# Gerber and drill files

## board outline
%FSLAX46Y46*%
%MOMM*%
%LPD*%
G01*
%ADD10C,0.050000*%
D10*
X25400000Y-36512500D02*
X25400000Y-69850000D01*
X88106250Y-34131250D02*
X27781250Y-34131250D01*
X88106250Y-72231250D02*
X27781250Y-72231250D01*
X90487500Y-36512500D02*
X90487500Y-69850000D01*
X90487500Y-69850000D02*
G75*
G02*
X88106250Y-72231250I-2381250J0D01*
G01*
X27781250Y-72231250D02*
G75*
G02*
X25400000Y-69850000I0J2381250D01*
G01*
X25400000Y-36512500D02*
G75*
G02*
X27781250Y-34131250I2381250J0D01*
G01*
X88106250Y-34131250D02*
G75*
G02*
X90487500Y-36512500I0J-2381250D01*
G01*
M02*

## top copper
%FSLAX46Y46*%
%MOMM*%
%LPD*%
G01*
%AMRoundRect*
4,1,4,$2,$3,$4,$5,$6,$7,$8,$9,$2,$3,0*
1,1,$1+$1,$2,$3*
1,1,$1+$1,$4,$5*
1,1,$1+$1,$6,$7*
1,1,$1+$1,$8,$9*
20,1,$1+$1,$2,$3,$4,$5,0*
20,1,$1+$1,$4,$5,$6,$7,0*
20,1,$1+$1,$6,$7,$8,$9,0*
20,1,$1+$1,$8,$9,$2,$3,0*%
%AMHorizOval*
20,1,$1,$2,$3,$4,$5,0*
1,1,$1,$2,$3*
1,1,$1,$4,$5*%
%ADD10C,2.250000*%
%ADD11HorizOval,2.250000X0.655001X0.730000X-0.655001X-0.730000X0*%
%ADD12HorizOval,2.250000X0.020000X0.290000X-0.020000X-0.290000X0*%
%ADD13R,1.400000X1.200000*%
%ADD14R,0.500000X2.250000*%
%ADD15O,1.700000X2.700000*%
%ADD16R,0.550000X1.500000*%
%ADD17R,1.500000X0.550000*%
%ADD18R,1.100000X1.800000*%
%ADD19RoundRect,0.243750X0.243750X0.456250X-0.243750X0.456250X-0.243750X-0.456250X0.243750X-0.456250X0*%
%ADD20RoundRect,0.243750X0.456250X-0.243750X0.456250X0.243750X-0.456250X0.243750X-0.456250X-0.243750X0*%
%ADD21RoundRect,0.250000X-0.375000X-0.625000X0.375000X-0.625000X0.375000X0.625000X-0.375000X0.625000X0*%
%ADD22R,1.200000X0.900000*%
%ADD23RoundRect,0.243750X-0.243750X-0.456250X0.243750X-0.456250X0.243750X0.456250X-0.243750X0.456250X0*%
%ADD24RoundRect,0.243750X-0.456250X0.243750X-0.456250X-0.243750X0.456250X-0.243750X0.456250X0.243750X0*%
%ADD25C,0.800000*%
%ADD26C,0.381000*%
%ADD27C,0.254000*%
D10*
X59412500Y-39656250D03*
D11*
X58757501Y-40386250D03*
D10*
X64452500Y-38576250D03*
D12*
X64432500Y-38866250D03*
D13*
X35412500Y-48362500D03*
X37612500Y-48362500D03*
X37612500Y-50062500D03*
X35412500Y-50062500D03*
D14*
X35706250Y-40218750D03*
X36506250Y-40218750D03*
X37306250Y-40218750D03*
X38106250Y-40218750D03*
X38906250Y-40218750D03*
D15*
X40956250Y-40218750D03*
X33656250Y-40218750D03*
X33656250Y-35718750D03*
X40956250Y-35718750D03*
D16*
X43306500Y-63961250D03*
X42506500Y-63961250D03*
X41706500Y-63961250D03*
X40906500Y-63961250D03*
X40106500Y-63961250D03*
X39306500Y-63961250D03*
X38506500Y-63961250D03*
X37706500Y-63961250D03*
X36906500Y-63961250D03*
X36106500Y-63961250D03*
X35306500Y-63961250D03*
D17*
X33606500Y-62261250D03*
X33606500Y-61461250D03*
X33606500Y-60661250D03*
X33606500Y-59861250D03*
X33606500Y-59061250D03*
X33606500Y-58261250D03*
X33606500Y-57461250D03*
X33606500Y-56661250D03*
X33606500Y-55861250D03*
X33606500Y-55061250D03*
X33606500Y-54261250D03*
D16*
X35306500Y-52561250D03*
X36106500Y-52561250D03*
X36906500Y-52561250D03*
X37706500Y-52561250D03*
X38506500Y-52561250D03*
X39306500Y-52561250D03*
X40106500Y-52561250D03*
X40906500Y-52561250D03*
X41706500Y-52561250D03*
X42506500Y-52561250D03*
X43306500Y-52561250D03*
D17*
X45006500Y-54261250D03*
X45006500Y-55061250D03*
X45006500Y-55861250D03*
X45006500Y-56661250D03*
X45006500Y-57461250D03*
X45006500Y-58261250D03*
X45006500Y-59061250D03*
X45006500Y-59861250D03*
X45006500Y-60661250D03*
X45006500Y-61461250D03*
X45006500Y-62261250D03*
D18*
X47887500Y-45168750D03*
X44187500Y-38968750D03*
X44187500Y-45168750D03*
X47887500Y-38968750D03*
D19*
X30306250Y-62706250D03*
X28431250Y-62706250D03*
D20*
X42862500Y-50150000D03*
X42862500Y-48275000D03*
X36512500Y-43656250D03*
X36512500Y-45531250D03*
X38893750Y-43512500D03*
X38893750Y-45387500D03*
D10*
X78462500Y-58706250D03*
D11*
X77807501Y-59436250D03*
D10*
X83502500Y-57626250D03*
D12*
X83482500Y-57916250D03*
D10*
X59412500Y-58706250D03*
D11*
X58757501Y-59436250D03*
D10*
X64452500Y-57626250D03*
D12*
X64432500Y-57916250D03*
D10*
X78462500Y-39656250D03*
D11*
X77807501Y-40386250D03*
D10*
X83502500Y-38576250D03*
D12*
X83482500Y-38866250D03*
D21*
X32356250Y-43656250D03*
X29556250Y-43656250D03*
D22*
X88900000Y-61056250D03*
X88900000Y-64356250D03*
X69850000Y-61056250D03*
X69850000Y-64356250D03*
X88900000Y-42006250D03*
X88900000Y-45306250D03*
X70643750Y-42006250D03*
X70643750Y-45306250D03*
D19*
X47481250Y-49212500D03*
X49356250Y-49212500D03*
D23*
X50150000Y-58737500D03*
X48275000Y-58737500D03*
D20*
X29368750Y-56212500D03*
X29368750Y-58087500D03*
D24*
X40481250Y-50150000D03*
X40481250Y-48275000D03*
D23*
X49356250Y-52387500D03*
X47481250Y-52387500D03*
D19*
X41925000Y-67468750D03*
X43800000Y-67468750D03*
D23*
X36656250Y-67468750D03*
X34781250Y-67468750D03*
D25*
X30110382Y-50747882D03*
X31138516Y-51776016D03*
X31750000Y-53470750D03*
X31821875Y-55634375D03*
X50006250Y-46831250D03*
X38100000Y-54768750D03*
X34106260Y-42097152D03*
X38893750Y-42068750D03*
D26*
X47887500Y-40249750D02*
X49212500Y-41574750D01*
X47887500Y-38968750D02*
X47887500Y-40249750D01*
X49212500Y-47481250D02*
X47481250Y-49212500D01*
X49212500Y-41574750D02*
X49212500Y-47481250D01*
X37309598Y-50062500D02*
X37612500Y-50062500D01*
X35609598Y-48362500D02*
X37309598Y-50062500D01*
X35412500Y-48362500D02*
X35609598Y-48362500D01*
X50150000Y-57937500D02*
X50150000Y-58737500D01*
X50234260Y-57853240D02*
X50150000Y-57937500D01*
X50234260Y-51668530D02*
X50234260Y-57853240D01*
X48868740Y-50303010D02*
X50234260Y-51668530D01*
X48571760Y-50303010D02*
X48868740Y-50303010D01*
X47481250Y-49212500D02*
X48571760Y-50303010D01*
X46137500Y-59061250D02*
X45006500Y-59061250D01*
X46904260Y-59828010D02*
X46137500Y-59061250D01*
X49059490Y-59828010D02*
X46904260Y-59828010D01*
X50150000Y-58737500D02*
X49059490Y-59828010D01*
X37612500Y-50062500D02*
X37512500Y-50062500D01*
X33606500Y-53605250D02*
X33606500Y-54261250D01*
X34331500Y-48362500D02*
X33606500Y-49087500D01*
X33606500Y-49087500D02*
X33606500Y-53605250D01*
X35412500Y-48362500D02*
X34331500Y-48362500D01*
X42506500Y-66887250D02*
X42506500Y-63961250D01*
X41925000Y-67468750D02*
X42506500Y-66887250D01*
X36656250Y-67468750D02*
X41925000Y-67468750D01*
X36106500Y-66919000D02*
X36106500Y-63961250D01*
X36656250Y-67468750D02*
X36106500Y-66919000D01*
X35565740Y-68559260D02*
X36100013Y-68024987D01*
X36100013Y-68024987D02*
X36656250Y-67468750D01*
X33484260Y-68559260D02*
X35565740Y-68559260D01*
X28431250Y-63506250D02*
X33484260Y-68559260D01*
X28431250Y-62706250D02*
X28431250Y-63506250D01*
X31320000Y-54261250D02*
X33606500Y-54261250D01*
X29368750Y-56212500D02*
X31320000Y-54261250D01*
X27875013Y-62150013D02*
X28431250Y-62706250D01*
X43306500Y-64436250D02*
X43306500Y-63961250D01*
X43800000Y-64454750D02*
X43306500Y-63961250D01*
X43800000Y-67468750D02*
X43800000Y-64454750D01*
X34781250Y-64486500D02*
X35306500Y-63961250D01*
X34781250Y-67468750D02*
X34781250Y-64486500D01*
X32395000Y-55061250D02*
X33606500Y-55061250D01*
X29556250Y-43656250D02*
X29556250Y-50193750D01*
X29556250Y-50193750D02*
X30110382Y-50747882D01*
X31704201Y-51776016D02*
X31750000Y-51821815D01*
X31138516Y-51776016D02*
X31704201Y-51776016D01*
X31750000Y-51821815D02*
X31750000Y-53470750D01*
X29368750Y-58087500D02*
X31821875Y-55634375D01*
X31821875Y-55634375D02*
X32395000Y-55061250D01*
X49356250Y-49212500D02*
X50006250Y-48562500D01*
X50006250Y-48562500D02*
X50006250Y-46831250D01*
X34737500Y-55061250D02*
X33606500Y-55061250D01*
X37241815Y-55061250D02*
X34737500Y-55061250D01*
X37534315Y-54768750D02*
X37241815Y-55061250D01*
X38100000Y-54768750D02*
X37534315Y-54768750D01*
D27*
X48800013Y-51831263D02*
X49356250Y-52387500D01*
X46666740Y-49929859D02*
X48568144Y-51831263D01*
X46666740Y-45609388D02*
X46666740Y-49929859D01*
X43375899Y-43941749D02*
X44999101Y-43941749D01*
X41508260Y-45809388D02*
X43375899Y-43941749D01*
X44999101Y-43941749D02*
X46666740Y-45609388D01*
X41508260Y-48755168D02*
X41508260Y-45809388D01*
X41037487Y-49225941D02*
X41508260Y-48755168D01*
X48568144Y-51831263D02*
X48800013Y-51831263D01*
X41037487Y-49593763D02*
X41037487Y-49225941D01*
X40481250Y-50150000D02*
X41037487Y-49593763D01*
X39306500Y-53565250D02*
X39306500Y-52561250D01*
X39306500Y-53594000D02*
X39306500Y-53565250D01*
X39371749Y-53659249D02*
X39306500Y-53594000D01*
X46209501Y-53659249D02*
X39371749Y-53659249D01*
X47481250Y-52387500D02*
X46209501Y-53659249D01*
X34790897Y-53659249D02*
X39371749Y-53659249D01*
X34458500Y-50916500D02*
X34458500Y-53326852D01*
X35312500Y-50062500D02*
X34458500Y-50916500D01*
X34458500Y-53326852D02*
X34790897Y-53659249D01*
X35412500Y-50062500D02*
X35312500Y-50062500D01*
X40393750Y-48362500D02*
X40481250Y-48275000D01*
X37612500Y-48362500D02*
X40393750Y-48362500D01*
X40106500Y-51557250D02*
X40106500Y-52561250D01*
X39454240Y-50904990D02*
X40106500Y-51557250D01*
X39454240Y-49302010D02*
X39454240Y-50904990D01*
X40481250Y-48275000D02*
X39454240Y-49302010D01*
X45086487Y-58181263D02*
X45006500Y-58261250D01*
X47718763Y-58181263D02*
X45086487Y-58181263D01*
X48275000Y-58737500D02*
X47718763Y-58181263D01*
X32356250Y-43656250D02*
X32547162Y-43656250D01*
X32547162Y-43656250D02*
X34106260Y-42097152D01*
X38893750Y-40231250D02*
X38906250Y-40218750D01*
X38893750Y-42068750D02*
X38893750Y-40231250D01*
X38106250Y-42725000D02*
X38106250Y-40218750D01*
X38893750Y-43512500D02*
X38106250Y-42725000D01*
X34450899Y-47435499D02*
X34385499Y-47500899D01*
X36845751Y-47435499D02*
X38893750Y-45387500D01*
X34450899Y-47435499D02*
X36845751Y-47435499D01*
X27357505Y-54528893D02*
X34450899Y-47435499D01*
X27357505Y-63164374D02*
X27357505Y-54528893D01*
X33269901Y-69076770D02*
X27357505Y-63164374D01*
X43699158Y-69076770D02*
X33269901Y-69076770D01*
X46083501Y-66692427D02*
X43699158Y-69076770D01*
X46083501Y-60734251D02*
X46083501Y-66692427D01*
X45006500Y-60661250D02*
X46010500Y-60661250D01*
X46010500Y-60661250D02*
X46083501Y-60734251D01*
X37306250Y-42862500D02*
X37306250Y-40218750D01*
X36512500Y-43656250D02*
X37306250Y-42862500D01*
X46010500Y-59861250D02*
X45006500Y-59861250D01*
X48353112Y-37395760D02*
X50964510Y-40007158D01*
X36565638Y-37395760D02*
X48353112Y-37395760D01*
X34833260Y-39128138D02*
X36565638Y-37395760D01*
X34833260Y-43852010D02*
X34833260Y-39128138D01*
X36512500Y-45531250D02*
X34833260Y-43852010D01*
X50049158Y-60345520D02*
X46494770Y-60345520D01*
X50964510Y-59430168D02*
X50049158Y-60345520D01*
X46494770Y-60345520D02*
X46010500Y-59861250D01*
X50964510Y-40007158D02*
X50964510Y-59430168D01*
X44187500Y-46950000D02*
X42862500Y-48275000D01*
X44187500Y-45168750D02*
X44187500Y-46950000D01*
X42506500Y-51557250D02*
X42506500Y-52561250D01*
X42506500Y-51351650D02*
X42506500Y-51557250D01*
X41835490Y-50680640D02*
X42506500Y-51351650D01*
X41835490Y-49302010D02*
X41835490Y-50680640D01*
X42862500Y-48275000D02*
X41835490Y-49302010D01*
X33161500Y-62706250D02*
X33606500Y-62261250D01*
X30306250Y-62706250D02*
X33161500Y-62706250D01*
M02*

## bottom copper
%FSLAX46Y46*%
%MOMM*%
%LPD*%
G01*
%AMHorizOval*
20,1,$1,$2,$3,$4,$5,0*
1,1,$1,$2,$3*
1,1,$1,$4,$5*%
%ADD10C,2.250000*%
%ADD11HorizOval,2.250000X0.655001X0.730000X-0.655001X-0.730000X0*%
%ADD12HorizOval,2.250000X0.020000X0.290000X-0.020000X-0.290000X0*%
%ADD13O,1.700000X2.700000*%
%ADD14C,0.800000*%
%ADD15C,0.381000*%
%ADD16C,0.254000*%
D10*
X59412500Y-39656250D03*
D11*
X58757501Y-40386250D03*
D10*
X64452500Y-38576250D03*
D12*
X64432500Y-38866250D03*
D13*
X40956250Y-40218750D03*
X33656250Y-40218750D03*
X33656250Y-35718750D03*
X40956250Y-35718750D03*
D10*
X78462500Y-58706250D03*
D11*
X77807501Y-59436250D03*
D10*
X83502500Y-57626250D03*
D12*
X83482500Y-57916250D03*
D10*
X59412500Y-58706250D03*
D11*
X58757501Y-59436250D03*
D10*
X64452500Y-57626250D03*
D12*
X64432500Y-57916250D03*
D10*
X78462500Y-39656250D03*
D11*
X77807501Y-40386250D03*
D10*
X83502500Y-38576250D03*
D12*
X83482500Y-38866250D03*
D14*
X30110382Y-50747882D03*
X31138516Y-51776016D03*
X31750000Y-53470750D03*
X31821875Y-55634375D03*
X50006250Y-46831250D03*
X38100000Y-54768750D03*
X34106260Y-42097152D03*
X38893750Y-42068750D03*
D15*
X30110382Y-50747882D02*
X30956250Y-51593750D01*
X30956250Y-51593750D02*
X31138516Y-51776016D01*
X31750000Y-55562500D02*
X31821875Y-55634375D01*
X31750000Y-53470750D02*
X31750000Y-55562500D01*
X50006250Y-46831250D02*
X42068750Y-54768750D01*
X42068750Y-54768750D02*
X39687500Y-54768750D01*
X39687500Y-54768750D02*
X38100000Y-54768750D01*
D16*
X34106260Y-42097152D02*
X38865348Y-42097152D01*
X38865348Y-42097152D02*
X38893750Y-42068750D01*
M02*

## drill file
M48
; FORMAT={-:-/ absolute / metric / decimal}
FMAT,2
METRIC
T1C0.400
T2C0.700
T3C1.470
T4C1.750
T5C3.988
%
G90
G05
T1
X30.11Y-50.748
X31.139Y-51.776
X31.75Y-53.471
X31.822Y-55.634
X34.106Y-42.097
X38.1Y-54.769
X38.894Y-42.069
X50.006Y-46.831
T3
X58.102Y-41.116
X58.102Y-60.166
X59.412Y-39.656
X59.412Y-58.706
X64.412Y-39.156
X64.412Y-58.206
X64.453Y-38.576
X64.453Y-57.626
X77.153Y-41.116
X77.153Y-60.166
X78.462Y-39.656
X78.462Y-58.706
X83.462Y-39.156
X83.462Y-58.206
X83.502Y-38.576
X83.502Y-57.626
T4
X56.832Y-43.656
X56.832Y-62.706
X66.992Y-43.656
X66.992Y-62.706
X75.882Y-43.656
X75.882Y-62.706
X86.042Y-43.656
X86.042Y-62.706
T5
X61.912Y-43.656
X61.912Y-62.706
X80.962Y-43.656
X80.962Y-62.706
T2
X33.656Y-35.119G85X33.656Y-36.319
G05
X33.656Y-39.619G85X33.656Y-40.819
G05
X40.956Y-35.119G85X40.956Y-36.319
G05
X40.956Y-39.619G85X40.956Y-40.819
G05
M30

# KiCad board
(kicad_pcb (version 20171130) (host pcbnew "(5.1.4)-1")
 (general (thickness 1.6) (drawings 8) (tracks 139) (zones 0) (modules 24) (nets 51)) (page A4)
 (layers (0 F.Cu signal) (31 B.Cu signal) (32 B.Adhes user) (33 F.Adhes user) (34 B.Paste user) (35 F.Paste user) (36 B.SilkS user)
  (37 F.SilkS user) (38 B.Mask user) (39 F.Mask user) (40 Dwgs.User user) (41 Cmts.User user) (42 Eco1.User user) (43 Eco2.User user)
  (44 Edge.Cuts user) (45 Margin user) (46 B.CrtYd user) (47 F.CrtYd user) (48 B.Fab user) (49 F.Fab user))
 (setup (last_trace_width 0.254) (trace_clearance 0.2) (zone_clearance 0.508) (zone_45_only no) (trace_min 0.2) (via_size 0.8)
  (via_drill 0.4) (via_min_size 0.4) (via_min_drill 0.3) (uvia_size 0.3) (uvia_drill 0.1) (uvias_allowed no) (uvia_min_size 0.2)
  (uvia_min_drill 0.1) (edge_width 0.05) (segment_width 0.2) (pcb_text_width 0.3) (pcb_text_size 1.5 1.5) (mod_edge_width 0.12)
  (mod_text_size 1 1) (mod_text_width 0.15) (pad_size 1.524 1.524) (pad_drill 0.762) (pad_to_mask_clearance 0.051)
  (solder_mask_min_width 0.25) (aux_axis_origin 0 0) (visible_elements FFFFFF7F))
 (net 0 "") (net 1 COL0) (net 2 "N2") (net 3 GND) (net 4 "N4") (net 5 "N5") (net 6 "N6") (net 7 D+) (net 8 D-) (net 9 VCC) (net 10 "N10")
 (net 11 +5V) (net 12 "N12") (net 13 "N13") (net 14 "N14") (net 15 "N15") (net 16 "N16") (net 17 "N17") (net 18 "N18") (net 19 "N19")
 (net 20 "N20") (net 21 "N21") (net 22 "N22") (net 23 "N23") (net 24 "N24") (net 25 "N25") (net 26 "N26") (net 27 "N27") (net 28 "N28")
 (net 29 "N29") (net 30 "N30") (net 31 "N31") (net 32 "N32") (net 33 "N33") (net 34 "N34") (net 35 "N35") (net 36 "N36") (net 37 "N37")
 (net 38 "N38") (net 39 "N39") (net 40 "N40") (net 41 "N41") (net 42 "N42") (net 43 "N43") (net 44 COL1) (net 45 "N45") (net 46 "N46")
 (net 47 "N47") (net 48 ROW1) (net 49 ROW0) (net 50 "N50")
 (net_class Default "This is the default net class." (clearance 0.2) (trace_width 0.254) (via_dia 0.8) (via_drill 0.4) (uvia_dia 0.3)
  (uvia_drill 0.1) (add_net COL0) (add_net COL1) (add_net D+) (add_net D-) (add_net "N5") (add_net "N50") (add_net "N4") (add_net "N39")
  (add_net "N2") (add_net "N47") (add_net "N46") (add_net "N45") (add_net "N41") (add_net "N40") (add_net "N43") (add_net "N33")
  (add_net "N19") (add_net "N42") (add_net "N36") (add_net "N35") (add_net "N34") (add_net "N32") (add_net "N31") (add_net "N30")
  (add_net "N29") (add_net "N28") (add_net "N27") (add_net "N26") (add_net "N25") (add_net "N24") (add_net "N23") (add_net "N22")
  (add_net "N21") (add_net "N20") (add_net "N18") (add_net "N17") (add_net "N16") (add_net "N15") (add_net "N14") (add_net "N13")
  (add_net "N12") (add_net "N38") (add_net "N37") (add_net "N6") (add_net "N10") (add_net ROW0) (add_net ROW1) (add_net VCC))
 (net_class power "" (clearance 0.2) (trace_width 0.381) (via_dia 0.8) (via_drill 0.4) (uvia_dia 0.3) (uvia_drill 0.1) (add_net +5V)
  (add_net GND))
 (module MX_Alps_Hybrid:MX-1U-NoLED (layer F.Cu) (at 61.9125 43.65625)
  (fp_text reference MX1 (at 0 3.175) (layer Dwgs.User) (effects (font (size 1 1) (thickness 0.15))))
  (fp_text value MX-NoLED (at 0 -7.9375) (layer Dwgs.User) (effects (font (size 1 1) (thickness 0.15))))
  (pad "" np_thru_hole circle (at 5.08 0 48.0996) (size 1.75 1.75) (drill 1.75) (layers *.Cu *.Mask))
  (pad "" np_thru_hole circle (at -5.08 0 48.0996) (size 1.75 1.75) (drill 1.75) (layers *.Cu *.Mask))
  (pad 1 thru_hole circle (at -2.5 -4) (size 2.25 2.25) (drill 1.47) (layers *.Cu B.Mask) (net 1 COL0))
  (pad "" np_thru_hole circle (at 0 0) (size 3.9878 3.9878) (drill 3.9878) (layers *.Cu *.Mask))
  (pad 1 thru_hole oval (at -3.81 -2.54 48.0996) (size 4.211556 2.25) (drill 1.47 (offset 0.980778 0)) (layers *.Cu B.Mask) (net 1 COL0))
  (pad 2 thru_hole circle (at 2.54 -5.08) (size 2.25 2.25) (drill 1.47) (layers *.Cu B.Mask) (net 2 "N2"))
  (pad 2 thru_hole oval (at 2.5 -4.5 86.0548) (size 2.831378 2.25) (drill 1.47 (offset 0.290689 0)) (layers *.Cu B.Mask) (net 2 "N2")))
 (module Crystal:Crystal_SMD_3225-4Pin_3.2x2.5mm (layer F.Cu) (at 36.5125 49.2125)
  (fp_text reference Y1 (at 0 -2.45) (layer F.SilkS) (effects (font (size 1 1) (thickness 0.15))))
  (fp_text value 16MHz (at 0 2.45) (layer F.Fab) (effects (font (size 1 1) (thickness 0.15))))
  (pad 4 smd rect (at -1.1 -0.85) (size 1.4 1.2) (layers F.Cu F.Paste F.Mask) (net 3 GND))
  (pad 3 smd rect (at 1.1 -0.85) (size 1.4 1.2) (layers F.Cu F.Paste F.Mask) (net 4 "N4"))
  (pad 2 smd rect (at 1.1 0.85) (size 1.4 1.2) (layers F.Cu F.Paste F.Mask) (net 3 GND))
  (pad 1 smd rect (at -1.1 0.85) (size 1.4 1.2) (layers F.Cu F.Paste F.Mask) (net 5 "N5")))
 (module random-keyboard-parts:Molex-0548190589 (layer F.Cu) (at 37.30625 35.71875 270)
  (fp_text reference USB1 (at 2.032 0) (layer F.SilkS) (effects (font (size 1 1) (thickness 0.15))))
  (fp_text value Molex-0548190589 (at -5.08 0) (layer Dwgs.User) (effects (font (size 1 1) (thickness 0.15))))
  (pad 1 smd rect (at 4.5 1.6 270) (size 2.25 0.5) (layers F.Cu F.Paste F.Mask) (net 3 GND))
  (pad 2 smd rect (at 4.5 0.8 270) (size 2.25 0.5) (layers F.Cu F.Paste F.Mask) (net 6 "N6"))
  (pad 3 smd rect (at 4.5 0 270) (size 2.25 0.5) (layers F.Cu F.Paste F.Mask) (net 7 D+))
  (pad 4 smd rect (at 4.5 -0.8 270) (size 2.25 0.5) (layers F.Cu F.Paste F.Mask) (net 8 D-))
  (pad 5 smd rect (at 4.5 -1.6 270) (size 2.25 0.5) (layers F.Cu F.Paste F.Mask) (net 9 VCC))
  (pad 6 thru_hole oval (at 4.5 -3.65 270) (size 2.7 1.7) (drill oval 1.9 0.7) (layers *.Cu *.Mask) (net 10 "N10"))
  (pad 6 thru_hole oval (at 4.5 3.65 270) (size 2.7 1.7) (drill oval 1.9 0.7) (layers *.Cu *.Mask) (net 10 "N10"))
  (pad 6 thru_hole oval (at 0 3.65 270) (size 2.7 1.7) (drill oval 1.9 0.7) (layers *.Cu *.Mask) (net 10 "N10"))
  (pad 6 thru_hole oval (at 0 -3.65 270) (size 2.7 1.7) (drill oval 1.9 0.7) (layers *.Cu *.Mask) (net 10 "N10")))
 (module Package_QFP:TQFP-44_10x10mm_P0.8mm (layer F.Cu) (at 39.3065 58.26125 180)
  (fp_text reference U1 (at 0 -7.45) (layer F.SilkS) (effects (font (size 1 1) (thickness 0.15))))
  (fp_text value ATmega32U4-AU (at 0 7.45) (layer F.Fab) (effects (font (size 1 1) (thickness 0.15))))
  (pad 44 smd rect (at -4 -5.7 270) (size 1.5 0.55) (layers F.Cu F.Paste F.Mask) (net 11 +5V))
  (pad 43 smd rect (at -3.2 -5.7 270) (size 1.5 0.55) (layers F.Cu F.Paste F.Mask) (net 3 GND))
  (pad 42 smd rect (at -2.4 -5.7 270) (size 1.5 0.55) (layers F.Cu F.Paste F.Mask) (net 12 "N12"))
  (pad 41 smd rect (at -1.6 -5.7 270) (size 1.5 0.55) (layers F.Cu F.Paste F.Mask) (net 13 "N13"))
  (pad 40 smd rect (at -0.8 -5.7 270) (size 1.5 0.55) (layers F.Cu F.Paste F.Mask) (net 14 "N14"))
  (pad 39 smd rect (at 0 -5.7 270) (size 1.5 0.55) (layers F.Cu F.Paste F.Mask) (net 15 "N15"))
  (pad 38 smd rect (at 0.8 -5.7 270) (size 1.5 0.55) (layers F.Cu F.Paste F.Mask) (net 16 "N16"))
  (pad 37 smd rect (at 1.6 -5.7 270) (size 1.5 0.55) (layers F.Cu F.Paste F.Mask) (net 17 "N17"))
  (pad 36 smd rect (at 2.4 -5.7 270) (size 1.5 0.55) (layers F.Cu F.Paste F.Mask) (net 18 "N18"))
  (pad 35 smd rect (at 3.2 -5.7 270) (size 1.5 0.55) (layers F.Cu F.Paste F.Mask) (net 3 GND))
  (pad 34 smd rect (at 4 -5.7 270) (size 1.5 0.55) (layers F.Cu F.Paste F.Mask) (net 11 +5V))
  (pad 33 smd rect (at 5.7 -4 180) (size 1.5 0.55) (layers F.Cu F.Paste F.Mask) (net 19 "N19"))
  (pad 32 smd rect (at 5.7 -3.2 180) (size 1.5 0.55) (layers F.Cu F.Paste F.Mask) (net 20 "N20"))
  (pad 31 smd rect (at 5.7 -2.4 180) (size 1.5 0.55) (layers F.Cu F.Paste F.Mask) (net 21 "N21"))
  (pad 30 smd rect (at 5.7 -1.6 180) (size 1.5 0.55) (layers F.Cu F.Paste F.Mask) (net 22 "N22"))
  (pad 29 smd rect (at 5.7 -0.8 180) (size 1.5 0.55) (layers F.Cu F.Paste F.Mask) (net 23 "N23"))
  (pad 28 smd rect (at 5.7 0 180) (size 1.5 0.55) (layers F.Cu F.Paste F.Mask) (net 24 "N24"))
  (pad 27 smd rect (at 5.7 0.8 180) (size 1.5 0.55) (layers F.Cu F.Paste F.Mask) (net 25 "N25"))
  (pad 26 smd rect (at 5.7 1.6 180) (size 1.5 0.55) (layers F.Cu F.Paste F.Mask) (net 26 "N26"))
  (pad 25 smd rect (at 5.7 2.4 180) (size 1.5 0.55) (layers F.Cu F.Paste F.Mask) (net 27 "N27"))
  (pad 24 smd rect (at 5.7 3.2 180) (size 1.5 0.55) (layers F.Cu F.Paste F.Mask) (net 11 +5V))
  (pad 23 smd rect (at 5.7 4 180) (size 1.5 0.55) (layers F.Cu F.Paste F.Mask) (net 3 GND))
  (pad 22 smd rect (at 4 5.7 270) (size 1.5 0.55) (layers F.Cu F.Paste F.Mask) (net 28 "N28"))
  (pad 21 smd rect (at 3.2 5.7 270) (size 1.5 0.55) (layers F.Cu F.Paste F.Mask) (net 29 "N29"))
  (pad 20 smd rect (at 2.4 5.7 270) (size 1.5 0.55) (layers F.Cu F.Paste F.Mask) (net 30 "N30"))
  (pad 19 smd rect (at 1.6 5.7 270) (size 1.5 0.55) (layers F.Cu F.Paste F.Mask) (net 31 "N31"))
  (pad 18 smd rect (at 0.8 5.7 270) (size 1.5 0.55) (layers F.Cu F.Paste F.Mask) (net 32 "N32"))
  (pad 17 smd rect (at 0 5.7 270) (size 1.5 0.55) (layers F.Cu F.Paste F.Mask) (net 5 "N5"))
  (pad 16 smd rect (at -0.8 5.7 270) (size 1.5 0.55) (layers F.Cu F.Paste F.Mask) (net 4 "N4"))
  (pad 15 smd rect (at -1.6 5.7 270) (size 1.5 0.55) (layers F.Cu F.Paste F.Mask) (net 3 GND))
  (pad 14 smd rect (at -2.4 5.7 270) (size 1.5 0.55) (layers F.Cu F.Paste F.Mask) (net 11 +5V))
  (pad 13 smd rect (at -3.2 5.7 270) (size 1.5 0.55) (layers F.Cu F.Paste F.Mask) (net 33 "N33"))
  (pad 12 smd rect (at -4 5.7 270) (size 1.5 0.55) (layers F.Cu F.Paste F.Mask) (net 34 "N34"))
  (pad 11 smd rect (at -5.7 4 180) (size 1.5 0.55) (layers F.Cu F.Paste F.Mask) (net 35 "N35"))
  (pad 10 smd rect (at -5.7 3.2 180) (size 1.5 0.55) (layers F.Cu F.Paste F.Mask) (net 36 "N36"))
  (pad 9 smd rect (at -5.7 2.4 180) (size 1.5 0.55) (layers F.Cu F.Paste F.Mask) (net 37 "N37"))
  (pad 8 smd rect (at -5.7 1.6 180) (size 1.5 0.55) (layers F.Cu F.Paste F.Mask) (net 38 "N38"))
  (pad 7 smd rect (at -5.7 0.8 180) (size 1.5 0.55) (layers F.Cu F.Paste F.Mask) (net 11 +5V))
  (pad 6 smd rect (at -5.7 0 180) (size 1.5 0.55) (layers F.Cu F.Paste F.Mask) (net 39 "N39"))
  (pad 5 smd rect (at -5.7 -0.8 180) (size 1.5 0.55) (layers F.Cu F.Paste F.Mask) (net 3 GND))
  (pad 4 smd rect (at -5.7 -1.6 180) (size 1.5 0.55) (layers F.Cu F.Paste F.Mask) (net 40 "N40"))
  (pad 3 smd rect (at -5.7 -2.4 180) (size 1.5 0.55) (layers F.Cu F.Paste F.Mask) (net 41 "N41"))
  (pad 2 smd rect (at -5.7 -3.2 180) (size 1.5 0.55) (layers F.Cu F.Paste F.Mask) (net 11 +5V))
  (pad 1 smd rect (at -5.7 -4 180) (size 1.5 0.55) (layers F.Cu F.Paste F.Mask) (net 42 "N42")))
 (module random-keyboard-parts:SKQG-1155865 (layer F.Cu) (at 46.0375 42.06875 90)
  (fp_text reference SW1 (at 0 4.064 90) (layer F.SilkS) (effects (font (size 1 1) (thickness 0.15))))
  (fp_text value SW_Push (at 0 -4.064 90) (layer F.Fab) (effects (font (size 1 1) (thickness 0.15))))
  (pad 4 smd rect (at -3.1 1.85 90) (size 1.8 1.1) (layers F.Cu F.Paste F.Mask))
  (pad 3 smd rect (at 3.1 -1.85 90) (size 1.8 1.1) (layers F.Cu F.Paste F.Mask))
  (pad 2 smd rect (at -3.1 -1.85 90) (size 1.8 1.1) (layers F.Cu F.Paste F.Mask) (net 33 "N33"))
  (pad 1 smd rect (at 3.1 1.85 90) (size 1.8 1.1) (layers F.Cu F.Paste F.Mask) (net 3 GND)))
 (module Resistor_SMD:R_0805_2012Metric (layer F.Cu) (at 29.36875 62.70625 180)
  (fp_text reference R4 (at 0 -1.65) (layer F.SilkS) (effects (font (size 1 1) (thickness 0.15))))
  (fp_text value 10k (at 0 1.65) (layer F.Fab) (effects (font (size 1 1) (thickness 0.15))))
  (pad 1 smd roundrect (at -0.9375 0 180) (size 0.975 1.4) (layers F.Cu F.Paste F.Mask) (roundrect_rratio 0.25) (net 19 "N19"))
  (pad 2 smd roundrect (at 0.9375 0 180) (size 0.975 1.4) (layers F.Cu F.Paste F.Mask) (roundrect_rratio 0.25) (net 3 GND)))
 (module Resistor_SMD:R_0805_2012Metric (layer F.Cu) (at 42.8625 49.2125 90)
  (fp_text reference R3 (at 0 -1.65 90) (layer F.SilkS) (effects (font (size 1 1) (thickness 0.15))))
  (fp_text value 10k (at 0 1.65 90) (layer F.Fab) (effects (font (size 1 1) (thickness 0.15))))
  (pad 1 smd roundrect (at -0.9375 0 90) (size 0.975 1.4) (layers F.Cu F.Paste F.Mask) (roundrect_rratio 0.25) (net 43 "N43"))
  (pad 2 smd roundrect (at 0.9375 0 90) (size 0.975 1.4) (layers F.Cu F.Paste F.Mask) (roundrect_rratio 0.25) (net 33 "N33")))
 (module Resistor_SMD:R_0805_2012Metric (layer F.Cu) (at 36.5125 44.59375 90)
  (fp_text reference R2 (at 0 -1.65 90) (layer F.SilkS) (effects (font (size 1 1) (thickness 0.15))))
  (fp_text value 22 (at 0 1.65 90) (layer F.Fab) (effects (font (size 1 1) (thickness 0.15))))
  (pad 2 smd roundrect (at 0.9375 0 90) (size 0.975 1.4) (layers F.Cu F.Paste F.Mask) (roundrect_rratio 0.25) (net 7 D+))
  (pad 1 smd roundrect (at -0.9375 0 90) (size 0.975 1.4) (layers F.Cu F.Paste F.Mask) (roundrect_rratio 0.25) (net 40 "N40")))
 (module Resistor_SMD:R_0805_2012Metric (layer F.Cu) (at 38.89375 44.45 90)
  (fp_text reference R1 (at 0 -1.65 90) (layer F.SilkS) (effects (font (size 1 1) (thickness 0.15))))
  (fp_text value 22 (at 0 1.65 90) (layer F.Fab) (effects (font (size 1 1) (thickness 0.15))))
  (pad 2 smd roundrect (at 0.9375 0 90) (size 0.975 1.4) (layers F.Cu F.Paste F.Mask) (roundrect_rratio 0.25) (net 8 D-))
  (pad 1 smd roundrect (at -0.9375 0 90) (size 0.975 1.4) (layers F.Cu F.Paste F.Mask) (roundrect_rratio 0.25) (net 41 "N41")))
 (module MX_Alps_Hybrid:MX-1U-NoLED (layer F.Cu) (at 80.9625 62.70625)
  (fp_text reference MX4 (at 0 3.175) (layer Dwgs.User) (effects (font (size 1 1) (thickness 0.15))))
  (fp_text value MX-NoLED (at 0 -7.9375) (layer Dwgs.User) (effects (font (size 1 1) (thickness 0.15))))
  (pad "" np_thru_hole circle (at 5.08 0 48.0996) (size 1.75 1.75) (drill 1.75) (layers *.Cu *.Mask))
  (pad "" np_thru_hole circle (at -5.08 0 48.0996) (size 1.75 1.75) (drill 1.75) (layers *.Cu *.Mask))
  (pad 1 thru_hole circle (at -2.5 -4) (size 2.25 2.25) (drill 1.47) (layers *.Cu B.Mask) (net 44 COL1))
  (pad "" np_thru_hole circle (at 0 0) (size 3.9878 3.9878) (drill 3.9878) (layers *.Cu *.Mask))
  (pad 1 thru_hole oval (at -3.81 -2.54 48.0996) (size 4.211556 2.25) (drill 1.47 (offset 0.980778 0)) (layers *.Cu B.Mask) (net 44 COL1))
  (pad 2 thru_hole circle (at 2.54 -5.08) (size 2.25 2.25) (drill 1.47) (layers *.Cu B.Mask) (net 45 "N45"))
  (pad 2 thru_hole oval (at 2.5 -4.5 86.0548) (size 2.831378 2.25) (drill 1.47 (offset 0.290689 0)) (layers *.Cu B.Mask) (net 45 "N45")))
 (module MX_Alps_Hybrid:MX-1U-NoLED (layer F.Cu) (at 61.9125 62.70625)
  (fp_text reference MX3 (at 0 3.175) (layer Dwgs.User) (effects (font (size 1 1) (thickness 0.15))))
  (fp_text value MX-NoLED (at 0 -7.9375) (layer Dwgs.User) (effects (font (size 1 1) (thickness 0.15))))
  (pad "" np_thru_hole circle (at 5.08 0 48.0996) (size 1.75 1.75) (drill 1.75) (layers *.Cu *.Mask))
  (pad "" np_thru_hole circle (at -5.08 0 48.0996) (size 1.75 1.75) (drill 1.75) (layers *.Cu *.Mask))
  (pad 1 thru_hole circle (at -2.5 -4) (size 2.25 2.25) (drill 1.47) (layers *.Cu B.Mask) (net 44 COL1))
  (pad "" np_thru_hole circle (at 0 0) (size 3.9878 3.9878) (drill 3.9878) (layers *.Cu *.Mask))
  (pad 1 thru_hole oval (at -3.81 -2.54 48.0996) (size 4.211556 2.25) (drill 1.47 (offset 0.980778 0)) (layers *.Cu B.Mask) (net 44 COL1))
  (pad 2 thru_hole circle (at 2.54 -5.08) (size 2.25 2.25) (drill 1.47) (layers *.Cu B.Mask) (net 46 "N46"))
  (pad 2 thru_hole oval (at 2.5 -4.5 86.0548) (size 2.831378 2.25) (drill 1.47 (offset 0.290689 0)) (layers *.Cu B.Mask) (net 46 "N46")))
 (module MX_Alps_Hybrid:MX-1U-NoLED (layer F.Cu) (at 80.9625 43.65625)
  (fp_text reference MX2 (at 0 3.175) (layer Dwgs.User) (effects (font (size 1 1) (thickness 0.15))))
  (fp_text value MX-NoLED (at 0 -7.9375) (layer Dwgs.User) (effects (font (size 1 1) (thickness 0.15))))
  (pad "" np_thru_hole circle (at 5.08 0 48.0996) (size 1.75 1.75) (drill 1.75) (layers *.Cu *.Mask))
  (pad "" np_thru_hole circle (at -5.08 0 48.0996) (size 1.75 1.75) (drill 1.75) (layers *.Cu *.Mask))
  (pad 1 thru_hole circle (at -2.5 -4) (size 2.25 2.25) (drill 1.47) (layers *.Cu B.Mask) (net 1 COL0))
  (pad "" np_thru_hole circle (at 0 0) (size 3.9878 3.9878) (drill 3.9878) (layers *.Cu *.Mask))
  (pad 1 thru_hole oval (at -3.81 -2.54 48.0996) (size 4.211556 2.25) (drill 1.47 (offset 0.980778 0)) (layers *.Cu B.Mask) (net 1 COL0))
  (pad 2 thru_hole circle (at 2.54 -5.08) (size 2.25 2.25) (drill 1.47) (layers *.Cu B.Mask) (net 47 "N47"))
  (pad 2 thru_hole oval (at 2.5 -4.5 86.0548) (size 2.831378 2.25) (drill 1.47 (offset 0.290689 0)) (layers *.Cu B.Mask) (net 47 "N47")))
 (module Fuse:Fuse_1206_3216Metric (layer F.Cu) (at 30.95625 43.65625)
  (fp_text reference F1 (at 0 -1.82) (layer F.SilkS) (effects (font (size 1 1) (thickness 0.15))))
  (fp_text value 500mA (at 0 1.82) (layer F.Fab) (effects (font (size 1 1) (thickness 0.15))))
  (pad 2 smd roundrect (at 1.4 0) (size 1.25 1.75) (layers F.Cu F.Paste F.Mask) (roundrect_rratio 0.2) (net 9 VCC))
  (pad 1 smd roundrect (at -1.4 0) (size 1.25 1.75) (layers F.Cu F.Paste F.Mask) (roundrect_rratio 0.2) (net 11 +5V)))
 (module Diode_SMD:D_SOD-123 (layer F.Cu) (at 88.9 62.70625 90)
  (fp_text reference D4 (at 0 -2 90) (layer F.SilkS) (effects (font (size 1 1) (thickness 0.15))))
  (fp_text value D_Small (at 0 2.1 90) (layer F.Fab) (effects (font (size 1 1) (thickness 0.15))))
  (pad 2 smd rect (at 1.65 0 90) (size 0.9 1.2) (layers F.Cu F.Paste F.Mask) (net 45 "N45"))
  (pad 1 smd rect (at -1.65 0 90) (size 0.9 1.2) (layers F.Cu F.Paste F.Mask) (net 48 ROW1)))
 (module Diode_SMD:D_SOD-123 (layer F.Cu) (at 69.85 62.70625 90)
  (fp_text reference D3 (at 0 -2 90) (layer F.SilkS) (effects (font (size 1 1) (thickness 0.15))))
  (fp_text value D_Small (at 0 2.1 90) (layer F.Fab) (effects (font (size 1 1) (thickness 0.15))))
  (pad 2 smd rect (at 1.65 0 90) (size 0.9 1.2) (layers F.Cu F.Paste F.Mask) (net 46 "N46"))
  (pad 1 smd rect (at -1.65 0 90) (size 0.9 1.2) (layers F.Cu F.Paste F.Mask) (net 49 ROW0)))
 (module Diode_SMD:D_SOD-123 (layer F.Cu) (at 88.9 43.65625 90)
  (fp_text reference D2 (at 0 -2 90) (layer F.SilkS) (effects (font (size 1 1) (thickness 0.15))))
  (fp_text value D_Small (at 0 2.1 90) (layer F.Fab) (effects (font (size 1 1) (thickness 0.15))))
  (pad 2 smd rect (at 1.65 0 90) (size 0.9 1.2) (layers F.Cu F.Paste F.Mask) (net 47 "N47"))
  (pad 1 smd rect (at -1.65 0 90) (size 0.9 1.2) (layers F.Cu F.Paste F.Mask) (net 48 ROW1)))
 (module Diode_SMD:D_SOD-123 (layer F.Cu) (at 70.64375 43.65625 90)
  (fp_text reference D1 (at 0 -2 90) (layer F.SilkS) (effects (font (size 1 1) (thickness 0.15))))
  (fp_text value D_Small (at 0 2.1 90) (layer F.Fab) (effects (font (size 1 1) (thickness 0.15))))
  (pad 2 smd rect (at 1.65 0 90) (size 0.9 1.2) (layers F.Cu F.Paste F.Mask) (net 2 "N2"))
  (pad 1 smd rect (at -1.65 0 90) (size 0.9 1.2) (layers F.Cu F.Paste F.Mask) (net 49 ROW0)))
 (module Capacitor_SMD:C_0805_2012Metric (layer F.Cu) (at 48.41875 49.2125 180)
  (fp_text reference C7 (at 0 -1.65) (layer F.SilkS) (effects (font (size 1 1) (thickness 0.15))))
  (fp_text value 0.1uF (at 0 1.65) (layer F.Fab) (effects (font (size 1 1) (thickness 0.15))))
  (pad 2 smd roundrect (at 0.9375 0 180) (size 0.975 1.4) (layers F.Cu F.Paste F.Mask) (roundrect_rratio 0.25) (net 3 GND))
  (pad 1 smd roundrect (at -0.9375 0 180) (size 0.975 1.4) (layers F.Cu F.Paste F.Mask) (roundrect_rratio 0.25) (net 11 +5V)))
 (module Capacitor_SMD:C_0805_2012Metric (layer F.Cu) (at 49.2125 58.7375)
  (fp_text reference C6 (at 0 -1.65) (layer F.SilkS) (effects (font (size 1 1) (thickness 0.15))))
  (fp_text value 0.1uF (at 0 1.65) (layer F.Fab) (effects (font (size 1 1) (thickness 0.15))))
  (pad 2 smd roundrect (at 0.9375 0) (size 0.975 1.4) (layers F.Cu F.Paste F.Mask) (roundrect_rratio 0.25) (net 3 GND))
  (pad 1 smd roundrect (at -0.9375 0) (size 0.975 1.4) (layers F.Cu F.Paste F.Mask) (roundrect_rratio 0.25) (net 39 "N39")))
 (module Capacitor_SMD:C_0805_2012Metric (layer F.Cu) (at 29.36875 57.15 90)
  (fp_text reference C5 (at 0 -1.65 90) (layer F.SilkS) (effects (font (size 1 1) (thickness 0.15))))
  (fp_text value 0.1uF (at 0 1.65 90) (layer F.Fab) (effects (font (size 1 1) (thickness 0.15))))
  (pad 2 smd roundrect (at 0.9375 0 90) (size 0.975 1.4) (layers F.Cu F.Paste F.Mask) (roundrect_rratio 0.25) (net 3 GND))
  (pad 1 smd roundrect (at -0.9375 0 90) (size 0.975 1.4) (layers F.Cu F.Paste F.Mask) (roundrect_rratio 0.25) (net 11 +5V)))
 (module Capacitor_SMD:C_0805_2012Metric (layer F.Cu) (at 40.48125 49.2125 270)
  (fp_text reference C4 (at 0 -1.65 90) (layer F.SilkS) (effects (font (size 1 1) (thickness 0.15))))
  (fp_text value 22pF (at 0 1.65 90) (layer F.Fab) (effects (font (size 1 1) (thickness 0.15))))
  (pad 2 smd roundrect (at 0.9375 0 270) (size 0.975 1.4) (layers F.Cu F.Paste F.Mask) (roundrect_rratio 0.25) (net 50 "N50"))
  (pad 1 smd roundrect (at -0.9375 0 270) (size 0.975 1.4) (layers F.Cu F.Paste F.Mask) (roundrect_rratio 0.25) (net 4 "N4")))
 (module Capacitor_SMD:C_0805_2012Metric (layer F.Cu) (at 48.41875 52.3875)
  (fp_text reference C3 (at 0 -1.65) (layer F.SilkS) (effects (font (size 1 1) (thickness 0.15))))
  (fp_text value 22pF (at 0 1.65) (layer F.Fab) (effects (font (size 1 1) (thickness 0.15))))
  (pad 2 smd roundrect (at 0.9375 0) (size 0.975 1.4) (layers F.Cu F.Paste F.Mask) (roundrect_rratio 0.25) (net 50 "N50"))
  (pad 1 smd roundrect (at -0.9375 0) (size 0.975 1.4) (layers F.Cu F.Paste F.Mask) (roundrect_rratio 0.25) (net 5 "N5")))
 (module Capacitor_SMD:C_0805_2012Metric (layer F.Cu) (at 42.8625 67.46875 180)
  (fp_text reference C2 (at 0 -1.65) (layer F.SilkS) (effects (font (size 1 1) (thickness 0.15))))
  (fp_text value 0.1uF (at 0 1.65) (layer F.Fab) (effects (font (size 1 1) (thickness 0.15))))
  (pad 2 smd roundrect (at 0.9375 0 180) (size 0.975 1.4) (layers F.Cu F.Paste F.Mask) (roundrect_rratio 0.25) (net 3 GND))
  (pad 1 smd roundrect (at -0.9375 0 180) (size 0.975 1.4) (layers F.Cu F.Paste F.Mask) (roundrect_rratio 0.25) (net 11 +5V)))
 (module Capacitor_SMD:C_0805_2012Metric (layer F.Cu) (at 35.71875 67.46875)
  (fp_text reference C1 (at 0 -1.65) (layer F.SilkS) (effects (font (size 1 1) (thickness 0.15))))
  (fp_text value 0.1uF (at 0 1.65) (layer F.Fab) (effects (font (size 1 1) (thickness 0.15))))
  (pad 2 smd roundrect (at 0.9375 0) (size 0.975 1.4) (layers F.Cu F.Paste F.Mask) (roundrect_rratio 0.25) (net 3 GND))
  (pad 1 smd roundrect (at -0.9375 0) (size 0.975 1.4) (layers F.Cu F.Paste F.Mask) (roundrect_rratio 0.25) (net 11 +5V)))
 (gr_line (start 25.4 36.5125) (end 25.4 69.85) (layer Edge.Cuts) (width 0.05))
 (gr_line (start 88.10625 34.13125) (end 27.78125 34.13125) (layer Edge.Cuts) (width 0.05))
 (gr_line (start 88.10625 72.23125) (end 27.78125 72.23125) (layer Edge.Cuts) (width 0.05))
 (gr_line (start 90.4875 36.5125) (end 90.4875 69.85) (layer Edge.Cuts) (width 0.05))
 (gr_arc (start 88.10625 69.85) (end 88.10625 72.23125) (angle -90) (layer Edge.Cuts) (width 0.05))
 (gr_arc (start 27.78125 69.85) (end 25.4 69.85) (angle -90) (layer Edge.Cuts) (width 0.05))
 (gr_arc (start 27.78125 36.5125) (end 27.78125 34.13125) (angle -90) (layer Edge.Cuts) (width 0.05))
 (gr_arc (start 88.10625 36.5125) (end 90.4875 36.5125) (angle -90) (layer Edge.Cuts) (width 0.05))
 (segment (start 47.8875 40.24975) (end 49.2125 41.57475) (width 0.381) (layer F.Cu) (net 3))
 (segment (start 47.8875 38.96875) (end 47.8875 40.24975) (width 0.381) (layer F.Cu) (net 3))
 (segment (start 49.2125 47.48125) (end 47.48125 49.2125) (width 0.381) (layer F.Cu) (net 3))
 (segment (start 49.2125 41.57475) (end 49.2125 47.48125) (width 0.381) (layer F.Cu) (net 3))
 (segment (start 37.309598 50.0625) (end 37.6125 50.0625) (width 0.381) (layer F.Cu) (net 3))
 (segment (start 35.609598 48.3625) (end 37.309598 50.0625) (width 0.381) (layer F.Cu) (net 3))
 (segment (start 35.4125 48.3625) (end 35.609598 48.3625) (width 0.381) (layer F.Cu) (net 3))
 (segment (start 50.15 57.9375) (end 50.15 58.7375) (width 0.381) (layer F.Cu) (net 3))
 (segment (start 50.23426 57.85324) (end 50.15 57.9375) (width 0.381) (layer F.Cu) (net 3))
 (segment (start 50.23426 51.66853) (end 50.23426 57.85324) (width 0.381) (layer F.Cu) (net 3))
 (segment (start 48.86874 50.30301) (end 50.23426 51.66853) (width 0.381) (layer F.Cu) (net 3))
 (segment (start 48.57176 50.30301) (end 48.86874 50.30301) (width 0.381) (layer F.Cu) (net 3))
 (segment (start 47.48125 49.2125) (end 48.57176 50.30301) (width 0.381) (layer F.Cu) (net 3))
 (segment (start 46.1375 59.06125) (end 45.0065 59.06125) (width 0.381) (layer F.Cu) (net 3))
 (segment (start 46.90426 59.82801) (end 46.1375 59.06125) (width 0.381) (layer F.Cu) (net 3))
 (segment (start 49.05949 59.82801) (end 46.90426 59.82801) (width 0.381) (layer F.Cu) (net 3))
 (segment (start 50.15 58.7375) (end 49.05949 59.82801) (width 0.381) (layer F.Cu) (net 3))
 (segment (start 37.6125 50.0625) (end 37.5125 50.0625) (width 0.381) (layer F.Cu) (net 3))
 (segment (start 33.6065 53.60525) (end 33.6065 54.26125) (width 0.381) (layer F.Cu) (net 3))
 (segment (start 34.3315 48.3625) (end 33.6065 49.0875) (width 0.381) (layer F.Cu) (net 3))
 (segment (start 33.6065 49.0875) (end 33.6065 53.60525) (width 0.381) (layer F.Cu) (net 3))
 (segment (start 35.4125 48.3625) (end 34.3315 48.3625) (width 0.381) (layer F.Cu) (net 3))
 (segment (start 42.5065 66.88725) (end 42.5065 63.96125) (width 0.381) (layer F.Cu) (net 3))
 (segment (start 41.925 67.46875) (end 42.5065 66.88725) (width 0.381) (layer F.Cu) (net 3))
 (segment (start 36.65625 67.46875) (end 41.925 67.46875) (width 0.381) (layer F.Cu) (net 3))
 (segment (start 36.1065 66.919) (end 36.1065 63.96125) (width 0.381) (layer F.Cu) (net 3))
 (segment (start 36.65625 67.46875) (end 36.1065 66.919) (width 0.381) (layer F.Cu) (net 3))
 (segment (start 35.56574 68.55926) (end 36.100013 68.024987) (width 0.381) (layer F.Cu) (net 3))
 (segment (start 36.100013 68.024987) (end 36.65625 67.46875) (width 0.381) (layer F.Cu) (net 3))
 (segment (start 33.48426 68.55926) (end 35.56574 68.55926) (width 0.381) (layer F.Cu) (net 3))
 (segment (start 28.43125 63.50625) (end 33.48426 68.55926) (width 0.381) (layer F.Cu) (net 3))
 (segment (start 28.43125 62.70625) (end 28.43125 63.50625) (width 0.381) (layer F.Cu) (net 3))
 (segment (start 31.32 54.26125) (end 33.6065 54.26125) (width 0.381) (layer F.Cu) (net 3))
 (segment (start 29.36875 56.2125) (end 31.32 54.26125) (width 0.381) (layer F.Cu) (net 3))
 (segment (start 27.875013 62.150013) (end 28.43125 62.70625) (width 0.381) (layer F.Cu) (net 3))
 (segment (start 43.3065 64.43625) (end 43.3065 63.96125) (width 0.381) (layer F.Cu) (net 11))
 (segment (start 43.8 64.45475) (end 43.3065 63.96125) (width 0.381) (layer F.Cu) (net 11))
 (segment (start 43.8 67.46875) (end 43.8 64.45475) (width 0.381) (layer F.Cu) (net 11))
 (segment (start 34.78125 64.4865) (end 35.3065 63.96125) (width 0.381) (layer F.Cu) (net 11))
 (segment (start 34.78125 67.46875) (end 34.78125 64.4865) (width 0.381) (layer F.Cu) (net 11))
 (segment (start 32.395 55.06125) (end 33.6065 55.06125) (width 0.381) (layer F.Cu) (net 11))
 (segment (start 29.55625 43.65625) (end 29.55625 50.19375) (width 0.381) (layer F.Cu) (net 11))
 (via (at 30.110382 50.747882) (size 0.8) (drill 0.4) (layers F.Cu B.Cu) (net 11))
 (segment (start 29.55625 50.19375) (end 30.110382 50.747882) (width 0.381) (layer F.Cu) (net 11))
 (segment (start 30.110382 50.747882) (end 30.95625 51.59375) (width 0.381) (layer B.Cu) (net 11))
 (via (at 31.138516 51.776016) (size 0.8) (drill 0.4) (layers F.Cu B.Cu) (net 11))
 (segment (start 30.95625 51.59375) (end 31.138516 51.776016) (width 0.381) (layer B.Cu) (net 11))
 (segment (start 31.704201 51.776016) (end 31.75 51.821815) (width 0.381) (layer F.Cu) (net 11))
 (segment (start 31.138516 51.776016) (end 31.704201 51.776016) (width 0.381) (layer F.Cu) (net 11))
 (via (at 31.75 53.47075) (size 0.8) (drill 0.4) (layers F.Cu B.Cu) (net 11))
 (segment (start 31.75 51.821815) (end 31.75 53.47075) (width 0.381) (layer F.Cu) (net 11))
 (segment (start 31.75 55.5625) (end 31.821875 55.634375) (width 0.381) (layer B.Cu) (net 11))
 (segment (start 31.75 53.47075) (end 31.75 55.5625) (width 0.381) (layer B.Cu) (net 11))
 (via (at 31.821875 55.634375) (size 0.8) (drill 0.4) (layers F.Cu B.Cu) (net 11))
 (segment (start 29.36875 58.0875) (end 31.821875 55.634375) (width 0.381) (layer F.Cu) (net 11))
 (segment (start 31.821875 55.634375) (end 32.395 55.06125) (width 0.381) (layer F.Cu) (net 11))
 (via (at 50.00625 46.83125) (size 0.8) (drill 0.4) (layers F.Cu B.Cu) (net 11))
 (segment (start 49.35625 49.2125) (end 50.00625 48.5625) (width 0.381) (layer F.Cu) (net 11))
 (segment (start 50.00625 48.5625) (end 50.00625 46.83125) (width 0.381) (layer F.Cu) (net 11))
 (segment (start 50.00625 46.83125) (end 42.06875 54.76875) (width 0.381) (layer B.Cu) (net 11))
 (segment (start 42.06875 54.76875) (end 39.6875 54.76875) (width 0.381) (layer B.Cu) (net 11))
 (via (at 38.1 54.76875) (size 0.8) (drill 0.4) (layers F.Cu B.Cu) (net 11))
 (segment (start 39.6875 54.76875) (end 38.1 54.76875) (width 0.381) (layer B.Cu) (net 11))
 (segment (start 34.7375 55.06125) (end 33.6065 55.06125) (width 0.381) (layer F.Cu) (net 11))
 (segment (start 37.241815 55.06125) (end 34.7375 55.06125) (width 0.381) (layer F.Cu) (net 11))
 (segment (start 37.534315 54.76875) (end 37.241815 55.06125) (width 0.381) (layer F.Cu) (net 11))
 (segment (start 38.1 54.76875) (end 37.534315 54.76875) (width 0.381) (layer F.Cu) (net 11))
 (segment (start 48.800013 51.831263) (end 49.35625 52.3875) (width 0.254) (layer F.Cu) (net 50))
 (segment (start 46.66674 49.929859) (end 48.568144 51.831263) (width 0.254) (layer F.Cu) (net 50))
 (segment (start 46.66674 45.609388) (end 46.66674 49.929859) (width 0.254) (layer F.Cu) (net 50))
 (segment (start 43.375899 43.941749) (end 44.999101 43.941749) (width 0.254) (layer F.Cu) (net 50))
 (segment (start 41.50826 45.809388) (end 43.375899 43.941749) (width 0.254) (layer F.Cu) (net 50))
 (segment (start 44.999101 43.941749) (end 46.66674 45.609388) (width 0.254) (layer F.Cu) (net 50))
 (segment (start 41.50826 48.755168) (end 41.50826 45.809388) (width 0.254) (layer F.Cu) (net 50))
 (segment (start 41.037487 49.225941) (end 41.50826 48.755168) (width 0.254) (layer F.Cu) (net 50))
 (segment (start 48.568144 51.831263) (end 48.800013 51.831263) (width 0.254) (layer F.Cu) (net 50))
 (segment (start 41.037487 49.593763) (end 41.037487 49.225941) (width 0.254) (layer F.Cu) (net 50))
 (segment (start 40.48125 50.15) (end 41.037487 49.593763) (width 0.254) (layer F.Cu) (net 50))
 (segment (start 39.3065 53.56525) (end 39.3065 52.56125) (width 0.254) (layer F.Cu) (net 5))
 (segment (start 39.3065 53.594) (end 39.3065 53.56525) (width 0.254) (layer F.Cu) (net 5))
 (segment (start 39.371749 53.659249) (end 39.3065 53.594) (width 0.254) (layer F.Cu) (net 5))
 (segment (start 46.209501 53.659249) (end 39.371749 53.659249) (width 0.254) (layer F.Cu) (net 5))
 (segment (start 47.48125 52.3875) (end 46.209501 53.659249) (width 0.254) (layer F.Cu) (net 5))
 (segment (start 34.790897 53.659249) (end 39.371749 53.659249) (width 0.254) (layer F.Cu) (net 5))
 (segment (start 34.4585 50.9165) (end 34.4585 53.326852) (width 0.254) (layer F.Cu) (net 5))
 (segment (start 35.3125 50.0625) (end 34.4585 50.9165) (width 0.254) (layer F.Cu) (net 5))
 (segment (start 34.4585 53.326852) (end 34.790897 53.659249) (width 0.254) (layer F.Cu) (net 5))
 (segment (start 35.4125 50.0625) (end 35.3125 50.0625) (width 0.254) (layer F.Cu) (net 5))
 (segment (start 40.39375 48.3625) (end 40.48125 48.275) (width 0.254) (layer F.Cu) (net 4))
 (segment (start 37.6125 48.3625) (end 40.39375 48.3625) (width 0.254) (layer F.Cu) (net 4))
 (segment (start 40.1065 51.55725) (end 40.1065 52.56125) (width 0.254) (layer F.Cu) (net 4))
 (segment (start 39.45424 50.90499) (end 40.1065 51.55725) (width 0.254) (layer F.Cu) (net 4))
 (segment (start 39.45424 49.30201) (end 39.45424 50.90499) (width 0.254) (layer F.Cu) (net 4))
 (segment (start 40.48125 48.275) (end 39.45424 49.30201) (width 0.254) (layer F.Cu) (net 4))
 (segment (start 45.086487 58.181263) (end 45.0065 58.26125) (width 0.254) (layer F.Cu) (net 39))
 (segment (start 47.718763 58.181263) (end 45.086487 58.181263) (width 0.254) (layer F.Cu) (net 39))
 (segment (start 48.275 58.7375) (end 47.718763 58.181263) (width 0.254) (layer F.Cu) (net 39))
 (via (at 34.10626 42.097152) (size 0.8) (drill 0.4) (layers F.Cu B.Cu) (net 9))
 (segment (start 32.35625 43.65625) (end 32.547162 43.65625) (width 0.254) (layer F.Cu) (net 9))
 (segment (start 32.547162 43.65625) (end 34.10626 42.097152) (width 0.254) (layer F.Cu) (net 9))
 (via (at 38.89375 42.06875) (size 0.8) (drill 0.4) (layers F.Cu B.Cu) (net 9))
 (segment (start 34.10626 42.097152) (end 38.865348 42.097152) (width 0.254) (layer B.Cu) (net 9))
 (segment (start 38.865348 42.097152) (end 38.89375 42.06875) (width 0.254) (layer B.Cu) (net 9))
 (segment (start 38.89375 40.23125) (end 38.90625 40.21875) (width 0.254) (layer F.Cu) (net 9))
 (segment (start 38.89375 42.06875) (end 38.89375 40.23125) (width 0.254) (layer F.Cu) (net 9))
 (segment (start 38.10625 42.725) (end 38.10625 40.21875) (width 0.254) (layer F.Cu) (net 8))
 (segment (start 38.89375 43.5125) (end 38.10625 42.725) (width 0.254) (layer F.Cu) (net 8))
 (segment (start 34.450899 47.435499) (end 34.385499 47.500899) (width 0.254) (layer F.Cu) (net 41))
 (segment (start 36.845751 47.435499) (end 38.89375 45.3875) (width 0.254) (layer F.Cu) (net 41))
 (segment (start 34.450899 47.435499) (end 36.845751 47.435499) (width 0.254) (layer F.Cu) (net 41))
 (segment (start 27.357505 54.528893) (end 34.450899 47.435499) (width 0.254) (layer F.Cu) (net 41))
 (segment (start 27.357505 63.164374) (end 27.357505 54.528893) (width 0.254) (layer F.Cu) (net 41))
 (segment (start 33.269901 69.07677) (end 27.357505 63.164374) (width 0.254) (layer F.Cu) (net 41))
 (segment (start 43.699158 69.07677) (end 33.269901 69.07677) (width 0.254) (layer F.Cu) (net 41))
 (segment (start 46.083501 66.692427) (end 43.699158 69.07677) (width 0.254) (layer F.Cu) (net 41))
 (segment (start 46.083501 60.734251) (end 46.083501 66.692427) (width 0.254) (layer F.Cu) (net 41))
 (segment (start 45.0065 60.66125) (end 46.0105 60.66125) (width 0.254) (layer F.Cu) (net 41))
 (segment (start 46.0105 60.66125) (end 46.083501 60.734251) (width 0.254) (layer F.Cu) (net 41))
 (segment (start 37.30625 42.8625) (end 37.30625 40.21875) (width 0.254) (layer F.Cu) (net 7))
 (segment (start 36.5125 43.65625) (end 37.30625 42.8625) (width 0.254) (layer F.Cu) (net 7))
 (segment (start 46.0105 59.86125) (end 45.0065 59.86125) (width 0.254) (layer F.Cu) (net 40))
 (segment (start 48.353112 37.39576) (end 50.96451 40.007158) (width 0.254) (layer F.Cu) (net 40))
 (segment (start 36.565638 37.39576) (end 48.353112 37.39576) (width 0.254) (layer F.Cu) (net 40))
 (segment (start 34.83326 39.128138) (end 36.565638 37.39576) (width 0.254) (layer F.Cu) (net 40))
 (segment (start 34.83326 43.85201) (end 34.83326 39.128138) (width 0.254) (layer F.Cu) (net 40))
 (segment (start 36.5125 45.53125) (end 34.83326 43.85201) (width 0.254) (layer F.Cu) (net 40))
 (segment (start 50.049158 60.34552) (end 46.49477 60.34552) (width 0.254) (layer F.Cu) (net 40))
 (segment (start 50.96451 59.430168) (end 50.049158 60.34552) (width 0.254) (layer F.Cu) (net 40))
 (segment (start 46.49477 60.34552) (end 46.0105 59.86125) (width 0.254) (layer F.Cu) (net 40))
 (segment (start 50.96451 40.007158) (end 50.96451 59.430168) (width 0.254) (layer F.Cu) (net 40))
 (segment (start 44.1875 46.95) (end 42.8625 48.275) (width 0.254) (layer F.Cu) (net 33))
 (segment (start 44.1875 45.16875) (end 44.1875 46.95) (width 0.254) (layer F.Cu) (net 33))
 (segment (start 42.5065 51.55725) (end 42.5065 52.56125) (width 0.254) (layer F.Cu) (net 33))
 (segment (start 42.5065 51.35165) (end 42.5065 51.55725) (width 0.254) (layer F.Cu) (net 33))
 (segment (start 41.83549 50.68064) (end 42.5065 51.35165) (width 0.254) (layer F.Cu) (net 33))
 (segment (start 41.83549 49.30201) (end 41.83549 50.68064) (width 0.254) (layer F.Cu) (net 33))
 (segment (start 42.8625 48.275) (end 41.83549 49.30201) (width 0.254) (layer F.Cu) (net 33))
 (segment (start 33.1615 62.70625) (end 33.6065 62.26125) (width 0.254) (layer F.Cu) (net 19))
 (segment (start 30.30625 62.70625) (end 33.1615 62.70625) (width 0.254) (layer F.Cu) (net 19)))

